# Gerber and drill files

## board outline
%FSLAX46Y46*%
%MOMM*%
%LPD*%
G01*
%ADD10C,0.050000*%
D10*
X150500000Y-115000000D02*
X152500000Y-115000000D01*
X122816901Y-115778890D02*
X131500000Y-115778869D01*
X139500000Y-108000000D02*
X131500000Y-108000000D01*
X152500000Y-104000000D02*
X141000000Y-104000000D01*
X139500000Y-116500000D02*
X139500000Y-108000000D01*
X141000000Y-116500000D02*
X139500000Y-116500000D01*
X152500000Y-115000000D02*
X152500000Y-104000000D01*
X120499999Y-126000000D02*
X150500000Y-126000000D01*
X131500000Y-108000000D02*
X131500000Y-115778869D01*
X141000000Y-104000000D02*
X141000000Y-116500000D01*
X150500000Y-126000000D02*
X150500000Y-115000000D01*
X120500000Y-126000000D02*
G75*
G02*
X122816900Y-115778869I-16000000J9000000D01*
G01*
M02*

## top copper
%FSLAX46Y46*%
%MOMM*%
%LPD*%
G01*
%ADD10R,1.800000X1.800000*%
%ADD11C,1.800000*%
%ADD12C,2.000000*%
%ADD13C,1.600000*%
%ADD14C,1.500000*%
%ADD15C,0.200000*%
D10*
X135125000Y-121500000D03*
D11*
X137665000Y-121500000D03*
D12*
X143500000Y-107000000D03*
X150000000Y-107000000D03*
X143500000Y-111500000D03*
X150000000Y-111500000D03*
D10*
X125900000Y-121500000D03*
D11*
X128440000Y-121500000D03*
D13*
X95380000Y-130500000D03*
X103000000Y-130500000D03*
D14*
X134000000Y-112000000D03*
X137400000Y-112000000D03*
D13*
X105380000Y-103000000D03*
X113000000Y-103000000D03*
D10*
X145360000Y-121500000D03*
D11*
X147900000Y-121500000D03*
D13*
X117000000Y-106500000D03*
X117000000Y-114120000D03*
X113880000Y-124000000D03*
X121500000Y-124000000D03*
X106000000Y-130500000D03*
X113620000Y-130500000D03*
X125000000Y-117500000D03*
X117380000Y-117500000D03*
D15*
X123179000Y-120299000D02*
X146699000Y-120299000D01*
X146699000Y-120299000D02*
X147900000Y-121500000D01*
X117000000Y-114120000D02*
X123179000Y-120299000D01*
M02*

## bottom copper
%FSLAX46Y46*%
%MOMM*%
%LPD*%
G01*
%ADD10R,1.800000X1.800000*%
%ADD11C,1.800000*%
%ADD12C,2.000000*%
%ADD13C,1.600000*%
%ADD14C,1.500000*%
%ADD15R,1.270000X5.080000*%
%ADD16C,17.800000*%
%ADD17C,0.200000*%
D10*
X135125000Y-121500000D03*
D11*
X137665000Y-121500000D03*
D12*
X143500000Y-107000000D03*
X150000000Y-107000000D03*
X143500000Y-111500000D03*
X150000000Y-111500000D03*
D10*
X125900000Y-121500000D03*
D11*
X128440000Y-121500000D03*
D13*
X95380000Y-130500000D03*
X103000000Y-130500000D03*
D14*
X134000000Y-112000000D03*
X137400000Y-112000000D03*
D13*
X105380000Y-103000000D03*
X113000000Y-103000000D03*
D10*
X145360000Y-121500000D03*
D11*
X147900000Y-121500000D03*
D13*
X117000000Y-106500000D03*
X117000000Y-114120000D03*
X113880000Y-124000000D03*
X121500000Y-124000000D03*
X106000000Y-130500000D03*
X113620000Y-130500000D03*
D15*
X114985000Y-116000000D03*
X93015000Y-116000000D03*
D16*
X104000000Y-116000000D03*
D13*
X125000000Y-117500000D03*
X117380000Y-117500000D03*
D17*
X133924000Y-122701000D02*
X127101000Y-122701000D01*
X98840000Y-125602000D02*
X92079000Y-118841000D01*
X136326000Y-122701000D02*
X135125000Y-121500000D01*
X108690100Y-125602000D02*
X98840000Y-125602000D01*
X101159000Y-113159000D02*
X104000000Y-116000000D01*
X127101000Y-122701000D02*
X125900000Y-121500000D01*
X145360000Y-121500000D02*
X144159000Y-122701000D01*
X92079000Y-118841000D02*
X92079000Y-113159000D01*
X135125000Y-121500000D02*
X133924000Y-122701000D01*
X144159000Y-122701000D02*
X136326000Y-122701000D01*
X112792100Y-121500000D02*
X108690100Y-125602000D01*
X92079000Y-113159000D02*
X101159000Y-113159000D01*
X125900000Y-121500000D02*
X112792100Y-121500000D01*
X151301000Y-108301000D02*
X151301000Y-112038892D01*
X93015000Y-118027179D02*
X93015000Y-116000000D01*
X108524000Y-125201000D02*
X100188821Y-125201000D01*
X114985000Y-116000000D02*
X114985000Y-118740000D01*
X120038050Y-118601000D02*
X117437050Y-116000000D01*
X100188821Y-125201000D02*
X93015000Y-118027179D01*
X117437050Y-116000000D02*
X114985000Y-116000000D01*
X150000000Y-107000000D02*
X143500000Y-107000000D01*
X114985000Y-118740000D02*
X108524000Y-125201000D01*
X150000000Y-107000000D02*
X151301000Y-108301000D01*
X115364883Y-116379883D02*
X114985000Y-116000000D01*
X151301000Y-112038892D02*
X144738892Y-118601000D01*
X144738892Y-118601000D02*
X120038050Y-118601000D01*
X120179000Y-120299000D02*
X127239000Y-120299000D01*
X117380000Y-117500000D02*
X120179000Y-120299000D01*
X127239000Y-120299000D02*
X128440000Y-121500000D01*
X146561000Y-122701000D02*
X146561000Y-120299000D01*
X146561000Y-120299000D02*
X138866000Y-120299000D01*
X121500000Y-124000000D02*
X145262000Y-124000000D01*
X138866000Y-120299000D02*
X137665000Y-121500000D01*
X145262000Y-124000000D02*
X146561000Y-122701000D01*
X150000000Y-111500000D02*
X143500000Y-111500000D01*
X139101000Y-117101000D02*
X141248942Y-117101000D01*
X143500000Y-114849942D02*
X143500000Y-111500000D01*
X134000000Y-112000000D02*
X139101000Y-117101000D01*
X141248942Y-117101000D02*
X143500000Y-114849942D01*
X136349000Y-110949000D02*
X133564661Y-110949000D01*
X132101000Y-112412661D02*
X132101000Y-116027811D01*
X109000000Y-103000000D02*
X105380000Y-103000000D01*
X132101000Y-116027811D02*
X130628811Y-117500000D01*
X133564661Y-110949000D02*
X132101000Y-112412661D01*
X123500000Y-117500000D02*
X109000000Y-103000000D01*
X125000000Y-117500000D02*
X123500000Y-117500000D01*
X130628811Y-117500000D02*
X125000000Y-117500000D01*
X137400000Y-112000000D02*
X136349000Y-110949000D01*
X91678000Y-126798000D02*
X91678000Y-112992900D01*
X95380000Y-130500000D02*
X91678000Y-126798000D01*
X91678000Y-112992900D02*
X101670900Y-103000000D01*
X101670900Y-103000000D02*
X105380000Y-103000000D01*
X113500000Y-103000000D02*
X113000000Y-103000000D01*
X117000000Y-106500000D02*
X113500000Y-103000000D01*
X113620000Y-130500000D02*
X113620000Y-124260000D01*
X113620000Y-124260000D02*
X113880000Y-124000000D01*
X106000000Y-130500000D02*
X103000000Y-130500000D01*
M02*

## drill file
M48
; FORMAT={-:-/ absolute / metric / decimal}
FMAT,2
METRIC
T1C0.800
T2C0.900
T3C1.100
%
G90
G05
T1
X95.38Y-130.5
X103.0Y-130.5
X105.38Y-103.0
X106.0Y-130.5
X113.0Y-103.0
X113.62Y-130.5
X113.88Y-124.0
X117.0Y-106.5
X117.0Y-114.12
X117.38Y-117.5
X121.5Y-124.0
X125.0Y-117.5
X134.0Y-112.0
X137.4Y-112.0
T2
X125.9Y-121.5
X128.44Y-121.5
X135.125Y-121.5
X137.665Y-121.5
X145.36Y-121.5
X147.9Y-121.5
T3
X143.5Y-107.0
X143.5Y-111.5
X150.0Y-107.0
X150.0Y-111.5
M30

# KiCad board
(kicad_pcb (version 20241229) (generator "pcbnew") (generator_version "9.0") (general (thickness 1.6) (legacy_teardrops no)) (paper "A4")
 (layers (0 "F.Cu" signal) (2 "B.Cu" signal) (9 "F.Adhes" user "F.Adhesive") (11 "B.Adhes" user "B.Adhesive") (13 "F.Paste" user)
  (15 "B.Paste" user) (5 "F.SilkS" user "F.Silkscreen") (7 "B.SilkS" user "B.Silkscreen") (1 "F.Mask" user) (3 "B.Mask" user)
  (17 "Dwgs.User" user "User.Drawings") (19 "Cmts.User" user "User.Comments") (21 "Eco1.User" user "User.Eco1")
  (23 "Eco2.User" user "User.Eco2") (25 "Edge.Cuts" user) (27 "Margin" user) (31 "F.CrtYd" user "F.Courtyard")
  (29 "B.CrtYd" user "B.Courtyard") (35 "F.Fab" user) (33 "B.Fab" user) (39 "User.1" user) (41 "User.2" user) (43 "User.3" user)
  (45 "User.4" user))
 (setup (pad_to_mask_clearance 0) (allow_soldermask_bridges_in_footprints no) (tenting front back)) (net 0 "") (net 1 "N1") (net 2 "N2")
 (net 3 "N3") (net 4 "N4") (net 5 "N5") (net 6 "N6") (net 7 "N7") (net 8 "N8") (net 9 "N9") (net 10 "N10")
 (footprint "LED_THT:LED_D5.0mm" (layer "F.Cu") (at 135.125 121.5)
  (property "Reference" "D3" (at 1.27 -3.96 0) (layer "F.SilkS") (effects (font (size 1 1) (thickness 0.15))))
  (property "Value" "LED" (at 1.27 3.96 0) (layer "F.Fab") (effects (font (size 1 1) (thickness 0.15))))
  (pad "1" thru_hole rect (at 0 0) (size 1.8 1.8) (drill 0.9) (layers "*.Cu" "*.Mask") (remove_unused_layers no) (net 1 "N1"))
  (pad "2" thru_hole circle (at 2.54 0) (size 1.8 1.8) (drill 0.9) (layers "*.Cu" "*.Mask") (remove_unused_layers no) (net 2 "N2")))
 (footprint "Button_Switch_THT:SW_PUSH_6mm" (layer "F.Cu") (at 143.5 107)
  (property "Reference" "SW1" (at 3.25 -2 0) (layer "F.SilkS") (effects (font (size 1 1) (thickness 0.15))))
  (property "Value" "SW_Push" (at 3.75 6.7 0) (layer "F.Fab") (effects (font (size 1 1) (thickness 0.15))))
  (pad "1" thru_hole circle (at 0 0 90) (size 2 2) (drill 1.1) (layers "*.Cu" "*.Mask") (remove_unused_layers no) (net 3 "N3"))
  (pad "1" thru_hole circle (at 6.5 0 90) (size 2 2) (drill 1.1) (layers "*.Cu" "*.Mask") (remove_unused_layers no) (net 3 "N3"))
  (pad "2" thru_hole circle (at 0 4.5 90) (size 2 2) (drill 1.1) (layers "*.Cu" "*.Mask") (remove_unused_layers no) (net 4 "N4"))
  (pad "2" thru_hole circle (at 6.5 4.5 90) (size 2 2) (drill 1.1) (layers "*.Cu" "*.Mask") (remove_unused_layers no) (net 4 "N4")))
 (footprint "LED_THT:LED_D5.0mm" (layer "F.Cu") (at 125.9 121.5)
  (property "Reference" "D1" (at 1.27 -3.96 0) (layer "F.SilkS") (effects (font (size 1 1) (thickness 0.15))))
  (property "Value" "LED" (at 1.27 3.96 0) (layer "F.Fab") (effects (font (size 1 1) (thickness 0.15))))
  (pad "1" thru_hole rect (at 0 0) (size 1.8 1.8) (drill 0.9) (layers "*.Cu" "*.Mask") (remove_unused_layers no) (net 1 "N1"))
  (pad "2" thru_hole circle (at 2.54 0) (size 1.8 1.8) (drill 0.9) (layers "*.Cu" "*.Mask") (remove_unused_layers no) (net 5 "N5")))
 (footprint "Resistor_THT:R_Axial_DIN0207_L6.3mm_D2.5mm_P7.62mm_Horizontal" (layer "F.Cu") (at 95.38 130.5)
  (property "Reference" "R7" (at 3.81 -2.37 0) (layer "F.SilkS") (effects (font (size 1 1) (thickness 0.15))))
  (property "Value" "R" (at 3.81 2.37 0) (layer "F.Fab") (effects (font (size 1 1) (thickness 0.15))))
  (pad "1" thru_hole circle (at 0 0) (size 1.6 1.6) (drill 0.8) (layers "*.Cu" "*.Mask") (remove_unused_layers no) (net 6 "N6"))
  (pad "2" thru_hole circle (at 7.62 0) (size 1.6 1.6) (drill 0.8) (layers "*.Cu" "*.Mask") (remove_unused_layers no) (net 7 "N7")))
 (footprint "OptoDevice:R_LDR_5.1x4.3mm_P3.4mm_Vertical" (layer "F.Cu") (at 134 112)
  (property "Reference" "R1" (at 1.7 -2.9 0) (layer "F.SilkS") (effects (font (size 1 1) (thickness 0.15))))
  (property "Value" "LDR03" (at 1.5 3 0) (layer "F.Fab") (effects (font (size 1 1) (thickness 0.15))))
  (pad "1" thru_hole circle (at 0 0) (size 1.5 1.5) (drill 0.8) (layers "*.Cu" "*.Mask") (remove_unused_layers no) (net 4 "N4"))
  (pad "2" thru_hole circle (at 3.4 0) (size 1.5 1.5) (drill 0.8) (layers "*.Cu" "*.Mask") (remove_unused_layers no) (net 6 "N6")))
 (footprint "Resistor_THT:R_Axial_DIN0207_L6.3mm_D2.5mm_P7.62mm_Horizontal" (layer "F.Cu") (at 105.38 103)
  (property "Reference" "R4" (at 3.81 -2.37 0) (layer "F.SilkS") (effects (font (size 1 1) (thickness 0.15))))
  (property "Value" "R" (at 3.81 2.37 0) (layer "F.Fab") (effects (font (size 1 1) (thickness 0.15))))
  (pad "1" thru_hole circle (at 0 0) (size 1.6 1.6) (drill 0.8) (layers "*.Cu" "*.Mask") (remove_unused_layers no) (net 6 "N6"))
  (pad "2" thru_hole circle (at 7.62 0) (size 1.6 1.6) (drill 0.8) (layers "*.Cu" "*.Mask") (remove_unused_layers no) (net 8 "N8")))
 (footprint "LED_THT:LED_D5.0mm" (layer "F.Cu") (at 145.36 121.5)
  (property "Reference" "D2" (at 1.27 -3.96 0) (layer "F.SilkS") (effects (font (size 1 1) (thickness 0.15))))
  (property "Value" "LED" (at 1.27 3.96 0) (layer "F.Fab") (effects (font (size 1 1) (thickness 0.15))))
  (pad "1" thru_hole rect (at 0 0) (size 1.8 1.8) (drill 0.9) (layers "*.Cu" "*.Mask") (remove_unused_layers no) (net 1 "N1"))
  (pad "2" thru_hole circle (at 2.54 0) (size 1.8 1.8) (drill 0.9) (layers "*.Cu" "*.Mask") (remove_unused_layers no) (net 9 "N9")))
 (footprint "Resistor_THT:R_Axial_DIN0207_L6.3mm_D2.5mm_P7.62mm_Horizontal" (layer "F.Cu") (at 117 106.5 -90)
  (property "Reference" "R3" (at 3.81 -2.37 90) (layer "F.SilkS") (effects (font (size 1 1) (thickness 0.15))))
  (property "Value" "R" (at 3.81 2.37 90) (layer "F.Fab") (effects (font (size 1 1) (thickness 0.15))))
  (pad "1" thru_hole circle (at 0 0 270) (size 1.6 1.6) (drill 0.8) (layers "*.Cu" "*.Mask") (remove_unused_layers no) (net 8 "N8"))
  (pad "2" thru_hole circle (at 7.62 0 270) (size 1.6 1.6) (drill 0.8) (layers "*.Cu" "*.Mask") (remove_unused_layers no) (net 9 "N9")))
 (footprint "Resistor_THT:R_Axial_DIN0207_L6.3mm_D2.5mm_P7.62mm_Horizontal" (layer "F.Cu") (at 113.88 124)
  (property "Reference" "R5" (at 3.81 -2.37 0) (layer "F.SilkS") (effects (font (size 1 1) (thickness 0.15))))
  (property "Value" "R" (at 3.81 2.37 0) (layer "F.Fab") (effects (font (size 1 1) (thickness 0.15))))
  (pad "1" thru_hole circle (at 0 0) (size 1.6 1.6) (drill 0.8) (layers "*.Cu" "*.Mask") (remove_unused_layers no) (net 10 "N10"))
  (pad "2" thru_hole circle (at 7.62 0) (size 1.6 1.6) (drill 0.8) (layers "*.Cu" "*.Mask") (remove_unused_layers no) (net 2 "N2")))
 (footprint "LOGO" (layer "F.Cu") (at 102.288197 116.516917)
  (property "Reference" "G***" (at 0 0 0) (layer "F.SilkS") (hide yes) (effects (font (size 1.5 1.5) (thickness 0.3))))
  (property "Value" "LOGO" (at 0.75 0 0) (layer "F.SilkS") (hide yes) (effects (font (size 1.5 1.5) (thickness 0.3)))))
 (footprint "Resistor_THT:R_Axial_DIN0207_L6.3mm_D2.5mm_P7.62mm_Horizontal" (layer "F.Cu") (at 106 130.5)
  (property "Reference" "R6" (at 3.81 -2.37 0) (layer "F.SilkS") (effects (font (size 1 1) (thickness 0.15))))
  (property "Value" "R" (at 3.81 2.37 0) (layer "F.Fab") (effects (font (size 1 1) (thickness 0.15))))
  (pad "1" thru_hole circle (at 0 0) (size 1.6 1.6) (drill 0.8) (layers "*.Cu" "*.Mask") (remove_unused_layers no) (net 7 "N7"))
  (pad "2" thru_hole circle (at 7.62 0) (size 1.6 1.6) (drill 0.8) (layers "*.Cu" "*.Mask") (remove_unused_layers no) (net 10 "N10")))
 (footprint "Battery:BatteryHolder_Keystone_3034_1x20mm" (layer "B.Cu") (at 104 116 180)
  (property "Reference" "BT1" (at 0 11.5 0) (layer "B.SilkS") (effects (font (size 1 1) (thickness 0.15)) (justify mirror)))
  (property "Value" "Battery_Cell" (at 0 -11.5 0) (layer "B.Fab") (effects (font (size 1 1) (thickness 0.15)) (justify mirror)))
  (pad "1" smd rect (at -10.985 0 180) (size 1.27 5.08) (layers "B.Cu" "B.Mask" "B.Paste") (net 3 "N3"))
  (pad "1" smd rect (at 10.985 0 180) (size 1.27 5.08) (layers "B.Cu" "B.Mask" "B.Paste") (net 3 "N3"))
  (pad "2" smd circle (at 0 0 180) (size 17.8 17.8) (layers "B.Cu" "B.Mask") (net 1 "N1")))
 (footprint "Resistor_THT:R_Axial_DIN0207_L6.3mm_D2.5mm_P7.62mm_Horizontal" (layer "B.Cu") (at 125 117.5 180)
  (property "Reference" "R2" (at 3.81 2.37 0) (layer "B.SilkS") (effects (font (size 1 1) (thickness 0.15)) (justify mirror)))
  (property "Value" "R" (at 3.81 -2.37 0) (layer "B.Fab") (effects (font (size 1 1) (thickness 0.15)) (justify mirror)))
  (pad "1" thru_hole circle (at 0 0 180) (size 1.6 1.6) (drill 0.8) (layers "*.Cu" "*.Mask") (remove_unused_layers no) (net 6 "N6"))
  (pad "2" thru_hole circle (at 7.62 0 180) (size 1.6 1.6) (drill 0.8) (layers "*.Cu" "*.Mask") (remove_unused_layers no) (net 5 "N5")))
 (gr_line (start 150.5 115) (end 152.5 115) (stroke (width 0.05) (type default)) (layer "Edge.Cuts"))
 (gr_line (start 122.816901 115.77889) (end 131.5 115.778869) (stroke (width 0.05) (type default)) (layer "Edge.Cuts"))
 (gr_line (start 139.5 108) (end 131.5 108) (stroke (width 0.05) (type default)) (layer "Edge.Cuts"))
 (gr_line (start 152.5 104) (end 141 104) (stroke (width 0.05) (type default)) (layer "Edge.Cuts"))
 (gr_line (start 139.5 116.5) (end 139.5 108) (stroke (width 0.05) (type default)) (layer "Edge.Cuts"))
 (gr_line (start 141 116.5) (end 139.5 116.5) (stroke (width 0.05) (type default)) (layer "Edge.Cuts"))
 (gr_line (start 152.5 115) (end 152.5 104) (stroke (width 0.05) (type default)) (layer "Edge.Cuts"))
 (gr_line (start 120.499999 126) (end 150.5 126) (stroke (width 0.05) (type default)) (layer "Edge.Cuts"))
 (gr_line (start 131.5 108) (end 131.5 115.778869) (stroke (width 0.05) (type default)) (layer "Edge.Cuts"))
 (gr_line (start 141 104) (end 141 116.5) (stroke (width 0.05) (type default)) (layer "Edge.Cuts"))
 (gr_line (start 150.5 126) (end 150.5 115) (stroke (width 0.05) (type default)) (layer "Edge.Cuts"))
 (gr_arc (start 120.5 126) (mid 86.59664 112.941711) (end 122.816901 115.778869) (stroke (width 0.05) (type default)) (layer "Edge.Cuts"))
 (segment (start 133.924 122.701) (end 127.101 122.701) (width 0.2) (layer "B.Cu") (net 1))
 (segment (start 98.84 125.602) (end 92.079 118.841) (width 0.2) (layer "B.Cu") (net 1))
 (segment (start 136.326 122.701) (end 135.125 121.5) (width 0.2) (layer "B.Cu") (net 1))
 (segment (start 108.6901 125.602) (end 98.84 125.602) (width 0.2) (layer "B.Cu") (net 1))
 (segment (start 101.159 113.159) (end 104 116) (width 0.2) (layer "B.Cu") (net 1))
 (segment (start 127.101 122.701) (end 125.9 121.5) (width 0.2) (layer "B.Cu") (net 1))
 (segment (start 145.36 121.5) (end 144.159 122.701) (width 0.2) (layer "B.Cu") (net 1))
 (segment (start 92.079 118.841) (end 92.079 113.159) (width 0.2) (layer "B.Cu") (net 1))
 (segment (start 135.125 121.5) (end 133.924 122.701) (width 0.2) (layer "B.Cu") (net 1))
 (segment (start 144.159 122.701) (end 136.326 122.701) (width 0.2) (layer "B.Cu") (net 1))
 (segment (start 112.7921 121.5) (end 108.6901 125.602) (width 0.2) (layer "B.Cu") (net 1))
 (segment (start 92.079 113.159) (end 101.159 113.159) (width 0.2) (layer "B.Cu") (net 1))
 (segment (start 125.9 121.5) (end 112.7921 121.5) (width 0.2) (layer "B.Cu") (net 1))
 (segment (start 151.301 108.301) (end 151.301 112.038892) (width 0.2) (layer "B.Cu") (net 3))
 (segment (start 93.015 118.027179) (end 93.015 116) (width 0.2) (layer "B.Cu") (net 3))
 (segment (start 108.524 125.201) (end 100.188821 125.201) (width 0.2) (layer "B.Cu") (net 3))
 (segment (start 114.985 116) (end 114.985 118.74) (width 0.2) (layer "B.Cu") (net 3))
 (segment (start 120.03805 118.601) (end 117.43705 116) (width 0.2) (layer "B.Cu") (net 3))
 (segment (start 100.188821 125.201) (end 93.015 118.027179) (width 0.2) (layer "B.Cu") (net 3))
 (segment (start 117.43705 116) (end 114.985 116) (width 0.2) (layer "B.Cu") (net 3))
 (segment (start 150 107) (end 143.5 107) (width 0.2) (layer "B.Cu") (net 3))
 (segment (start 114.985 118.74) (end 108.524 125.201) (width 0.2) (layer "B.Cu") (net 3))
 (segment (start 150 107) (end 151.301 108.301) (width 0.2) (layer "B.Cu") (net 3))
 (segment (start 115.364883 116.379883) (end 114.985 116) (width 0.2) (layer "B.Cu") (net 3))
 (segment (start 151.301 112.038892) (end 144.738892 118.601) (width 0.2) (layer "B.Cu") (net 3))
 (segment (start 144.738892 118.601) (end 120.03805 118.601) (width 0.2) (layer "B.Cu") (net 3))
 (segment (start 120.179 120.299) (end 127.239 120.299) (width 0.2) (layer "B.Cu") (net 5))
 (segment (start 117.38 117.5) (end 120.179 120.299) (width 0.2) (layer "B.Cu") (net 5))
 (segment (start 127.239 120.299) (end 128.44 121.5) (width 0.2) (layer "B.Cu") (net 5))
 (segment (start 123.179 120.299) (end 146.699 120.299) (width 0.2) (layer "F.Cu") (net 9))
 (segment (start 146.699 120.299) (end 147.9 121.5) (width 0.2) (layer "F.Cu") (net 9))
 (segment (start 117 114.12) (end 123.179 120.299) (width 0.2) (layer "F.Cu") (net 9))
 (segment (start 146.561 122.701) (end 146.561 120.299) (width 0.2) (layer "B.Cu") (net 2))
 (segment (start 146.561 120.299) (end 138.866 120.299) (width 0.2) (layer "B.Cu") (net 2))
 (segment (start 121.5 124) (end 145.262 124) (width 0.2) (layer "B.Cu") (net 2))
 (segment (start 138.866 120.299) (end 137.665 121.5) (width 0.2) (layer "B.Cu") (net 2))
 (segment (start 145.262 124) (end 146.561 122.701) (width 0.2) (layer "B.Cu") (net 2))
 (segment (start 150 111.5) (end 143.5 111.5) (width 0.2) (layer "B.Cu") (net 4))
 (segment (start 139.101 117.101) (end 141.248942 117.101) (width 0.2) (layer "B.Cu") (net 4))
 (segment (start 143.5 114.849942) (end 143.5 111.5) (width 0.2) (layer "B.Cu") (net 4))
 (segment (start 134 112) (end 139.101 117.101) (width 0.2) (layer "B.Cu") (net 4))
 (segment (start 141.248942 117.101) (end 143.5 114.849942) (width 0.2) (layer "B.Cu") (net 4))
 (segment (start 136.349 110.949) (end 133.564661 110.949) (width 0.2) (layer "B.Cu") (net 6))
 (segment (start 132.101 112.412661) (end 132.101 116.027811) (width 0.2) (layer "B.Cu") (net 6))
 (segment (start 109 103) (end 105.38 103) (width 0.2) (layer "B.Cu") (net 6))
 (segment (start 132.101 116.027811) (end 130.628811 117.5) (width 0.2) (layer "B.Cu") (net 6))
 (segment (start 133.564661 110.949) (end 132.101 112.412661) (width 0.2) (layer "B.Cu") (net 6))
 (segment (start 123.5 117.5) (end 109 103) (width 0.2) (layer "B.Cu") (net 6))
 (segment (start 125 117.5) (end 123.5 117.5) (width 0.2) (layer "B.Cu") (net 6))
 (segment (start 130.628811 117.5) (end 125 117.5) (width 0.2) (layer "B.Cu") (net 6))
 (segment (start 137.4 112) (end 136.349 110.949) (width 0.2) (layer "B.Cu") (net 6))
 (segment (start 91.678 126.798) (end 91.678 112.9929) (width 0.2) (layer "B.Cu") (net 6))
 (segment (start 95.38 130.5) (end 91.678 126.798) (width 0.2) (layer "B.Cu") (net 6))
 (segment (start 91.678 112.9929) (end 101.6709 103) (width 0.2) (layer "B.Cu") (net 6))
 (segment (start 101.6709 103) (end 105.38 103) (width 0.2) (layer "B.Cu") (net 6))
 (segment (start 113.5 103) (end 113 103) (width 0.2) (layer "B.Cu") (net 8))
 (segment (start 117 106.5) (end 113.5 103) (width 0.2) (layer "B.Cu") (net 8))
 (segment (start 113.62 130.5) (end 113.62 124.26) (width 0.2) (layer "B.Cu") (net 10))
 (segment (start 113.62 124.26) (end 113.88 124) (width 0.2) (layer "B.Cu") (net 10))
 (segment (start 106 130.5) (end 103 130.5) (width 0.2) (layer "B.Cu") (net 7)))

